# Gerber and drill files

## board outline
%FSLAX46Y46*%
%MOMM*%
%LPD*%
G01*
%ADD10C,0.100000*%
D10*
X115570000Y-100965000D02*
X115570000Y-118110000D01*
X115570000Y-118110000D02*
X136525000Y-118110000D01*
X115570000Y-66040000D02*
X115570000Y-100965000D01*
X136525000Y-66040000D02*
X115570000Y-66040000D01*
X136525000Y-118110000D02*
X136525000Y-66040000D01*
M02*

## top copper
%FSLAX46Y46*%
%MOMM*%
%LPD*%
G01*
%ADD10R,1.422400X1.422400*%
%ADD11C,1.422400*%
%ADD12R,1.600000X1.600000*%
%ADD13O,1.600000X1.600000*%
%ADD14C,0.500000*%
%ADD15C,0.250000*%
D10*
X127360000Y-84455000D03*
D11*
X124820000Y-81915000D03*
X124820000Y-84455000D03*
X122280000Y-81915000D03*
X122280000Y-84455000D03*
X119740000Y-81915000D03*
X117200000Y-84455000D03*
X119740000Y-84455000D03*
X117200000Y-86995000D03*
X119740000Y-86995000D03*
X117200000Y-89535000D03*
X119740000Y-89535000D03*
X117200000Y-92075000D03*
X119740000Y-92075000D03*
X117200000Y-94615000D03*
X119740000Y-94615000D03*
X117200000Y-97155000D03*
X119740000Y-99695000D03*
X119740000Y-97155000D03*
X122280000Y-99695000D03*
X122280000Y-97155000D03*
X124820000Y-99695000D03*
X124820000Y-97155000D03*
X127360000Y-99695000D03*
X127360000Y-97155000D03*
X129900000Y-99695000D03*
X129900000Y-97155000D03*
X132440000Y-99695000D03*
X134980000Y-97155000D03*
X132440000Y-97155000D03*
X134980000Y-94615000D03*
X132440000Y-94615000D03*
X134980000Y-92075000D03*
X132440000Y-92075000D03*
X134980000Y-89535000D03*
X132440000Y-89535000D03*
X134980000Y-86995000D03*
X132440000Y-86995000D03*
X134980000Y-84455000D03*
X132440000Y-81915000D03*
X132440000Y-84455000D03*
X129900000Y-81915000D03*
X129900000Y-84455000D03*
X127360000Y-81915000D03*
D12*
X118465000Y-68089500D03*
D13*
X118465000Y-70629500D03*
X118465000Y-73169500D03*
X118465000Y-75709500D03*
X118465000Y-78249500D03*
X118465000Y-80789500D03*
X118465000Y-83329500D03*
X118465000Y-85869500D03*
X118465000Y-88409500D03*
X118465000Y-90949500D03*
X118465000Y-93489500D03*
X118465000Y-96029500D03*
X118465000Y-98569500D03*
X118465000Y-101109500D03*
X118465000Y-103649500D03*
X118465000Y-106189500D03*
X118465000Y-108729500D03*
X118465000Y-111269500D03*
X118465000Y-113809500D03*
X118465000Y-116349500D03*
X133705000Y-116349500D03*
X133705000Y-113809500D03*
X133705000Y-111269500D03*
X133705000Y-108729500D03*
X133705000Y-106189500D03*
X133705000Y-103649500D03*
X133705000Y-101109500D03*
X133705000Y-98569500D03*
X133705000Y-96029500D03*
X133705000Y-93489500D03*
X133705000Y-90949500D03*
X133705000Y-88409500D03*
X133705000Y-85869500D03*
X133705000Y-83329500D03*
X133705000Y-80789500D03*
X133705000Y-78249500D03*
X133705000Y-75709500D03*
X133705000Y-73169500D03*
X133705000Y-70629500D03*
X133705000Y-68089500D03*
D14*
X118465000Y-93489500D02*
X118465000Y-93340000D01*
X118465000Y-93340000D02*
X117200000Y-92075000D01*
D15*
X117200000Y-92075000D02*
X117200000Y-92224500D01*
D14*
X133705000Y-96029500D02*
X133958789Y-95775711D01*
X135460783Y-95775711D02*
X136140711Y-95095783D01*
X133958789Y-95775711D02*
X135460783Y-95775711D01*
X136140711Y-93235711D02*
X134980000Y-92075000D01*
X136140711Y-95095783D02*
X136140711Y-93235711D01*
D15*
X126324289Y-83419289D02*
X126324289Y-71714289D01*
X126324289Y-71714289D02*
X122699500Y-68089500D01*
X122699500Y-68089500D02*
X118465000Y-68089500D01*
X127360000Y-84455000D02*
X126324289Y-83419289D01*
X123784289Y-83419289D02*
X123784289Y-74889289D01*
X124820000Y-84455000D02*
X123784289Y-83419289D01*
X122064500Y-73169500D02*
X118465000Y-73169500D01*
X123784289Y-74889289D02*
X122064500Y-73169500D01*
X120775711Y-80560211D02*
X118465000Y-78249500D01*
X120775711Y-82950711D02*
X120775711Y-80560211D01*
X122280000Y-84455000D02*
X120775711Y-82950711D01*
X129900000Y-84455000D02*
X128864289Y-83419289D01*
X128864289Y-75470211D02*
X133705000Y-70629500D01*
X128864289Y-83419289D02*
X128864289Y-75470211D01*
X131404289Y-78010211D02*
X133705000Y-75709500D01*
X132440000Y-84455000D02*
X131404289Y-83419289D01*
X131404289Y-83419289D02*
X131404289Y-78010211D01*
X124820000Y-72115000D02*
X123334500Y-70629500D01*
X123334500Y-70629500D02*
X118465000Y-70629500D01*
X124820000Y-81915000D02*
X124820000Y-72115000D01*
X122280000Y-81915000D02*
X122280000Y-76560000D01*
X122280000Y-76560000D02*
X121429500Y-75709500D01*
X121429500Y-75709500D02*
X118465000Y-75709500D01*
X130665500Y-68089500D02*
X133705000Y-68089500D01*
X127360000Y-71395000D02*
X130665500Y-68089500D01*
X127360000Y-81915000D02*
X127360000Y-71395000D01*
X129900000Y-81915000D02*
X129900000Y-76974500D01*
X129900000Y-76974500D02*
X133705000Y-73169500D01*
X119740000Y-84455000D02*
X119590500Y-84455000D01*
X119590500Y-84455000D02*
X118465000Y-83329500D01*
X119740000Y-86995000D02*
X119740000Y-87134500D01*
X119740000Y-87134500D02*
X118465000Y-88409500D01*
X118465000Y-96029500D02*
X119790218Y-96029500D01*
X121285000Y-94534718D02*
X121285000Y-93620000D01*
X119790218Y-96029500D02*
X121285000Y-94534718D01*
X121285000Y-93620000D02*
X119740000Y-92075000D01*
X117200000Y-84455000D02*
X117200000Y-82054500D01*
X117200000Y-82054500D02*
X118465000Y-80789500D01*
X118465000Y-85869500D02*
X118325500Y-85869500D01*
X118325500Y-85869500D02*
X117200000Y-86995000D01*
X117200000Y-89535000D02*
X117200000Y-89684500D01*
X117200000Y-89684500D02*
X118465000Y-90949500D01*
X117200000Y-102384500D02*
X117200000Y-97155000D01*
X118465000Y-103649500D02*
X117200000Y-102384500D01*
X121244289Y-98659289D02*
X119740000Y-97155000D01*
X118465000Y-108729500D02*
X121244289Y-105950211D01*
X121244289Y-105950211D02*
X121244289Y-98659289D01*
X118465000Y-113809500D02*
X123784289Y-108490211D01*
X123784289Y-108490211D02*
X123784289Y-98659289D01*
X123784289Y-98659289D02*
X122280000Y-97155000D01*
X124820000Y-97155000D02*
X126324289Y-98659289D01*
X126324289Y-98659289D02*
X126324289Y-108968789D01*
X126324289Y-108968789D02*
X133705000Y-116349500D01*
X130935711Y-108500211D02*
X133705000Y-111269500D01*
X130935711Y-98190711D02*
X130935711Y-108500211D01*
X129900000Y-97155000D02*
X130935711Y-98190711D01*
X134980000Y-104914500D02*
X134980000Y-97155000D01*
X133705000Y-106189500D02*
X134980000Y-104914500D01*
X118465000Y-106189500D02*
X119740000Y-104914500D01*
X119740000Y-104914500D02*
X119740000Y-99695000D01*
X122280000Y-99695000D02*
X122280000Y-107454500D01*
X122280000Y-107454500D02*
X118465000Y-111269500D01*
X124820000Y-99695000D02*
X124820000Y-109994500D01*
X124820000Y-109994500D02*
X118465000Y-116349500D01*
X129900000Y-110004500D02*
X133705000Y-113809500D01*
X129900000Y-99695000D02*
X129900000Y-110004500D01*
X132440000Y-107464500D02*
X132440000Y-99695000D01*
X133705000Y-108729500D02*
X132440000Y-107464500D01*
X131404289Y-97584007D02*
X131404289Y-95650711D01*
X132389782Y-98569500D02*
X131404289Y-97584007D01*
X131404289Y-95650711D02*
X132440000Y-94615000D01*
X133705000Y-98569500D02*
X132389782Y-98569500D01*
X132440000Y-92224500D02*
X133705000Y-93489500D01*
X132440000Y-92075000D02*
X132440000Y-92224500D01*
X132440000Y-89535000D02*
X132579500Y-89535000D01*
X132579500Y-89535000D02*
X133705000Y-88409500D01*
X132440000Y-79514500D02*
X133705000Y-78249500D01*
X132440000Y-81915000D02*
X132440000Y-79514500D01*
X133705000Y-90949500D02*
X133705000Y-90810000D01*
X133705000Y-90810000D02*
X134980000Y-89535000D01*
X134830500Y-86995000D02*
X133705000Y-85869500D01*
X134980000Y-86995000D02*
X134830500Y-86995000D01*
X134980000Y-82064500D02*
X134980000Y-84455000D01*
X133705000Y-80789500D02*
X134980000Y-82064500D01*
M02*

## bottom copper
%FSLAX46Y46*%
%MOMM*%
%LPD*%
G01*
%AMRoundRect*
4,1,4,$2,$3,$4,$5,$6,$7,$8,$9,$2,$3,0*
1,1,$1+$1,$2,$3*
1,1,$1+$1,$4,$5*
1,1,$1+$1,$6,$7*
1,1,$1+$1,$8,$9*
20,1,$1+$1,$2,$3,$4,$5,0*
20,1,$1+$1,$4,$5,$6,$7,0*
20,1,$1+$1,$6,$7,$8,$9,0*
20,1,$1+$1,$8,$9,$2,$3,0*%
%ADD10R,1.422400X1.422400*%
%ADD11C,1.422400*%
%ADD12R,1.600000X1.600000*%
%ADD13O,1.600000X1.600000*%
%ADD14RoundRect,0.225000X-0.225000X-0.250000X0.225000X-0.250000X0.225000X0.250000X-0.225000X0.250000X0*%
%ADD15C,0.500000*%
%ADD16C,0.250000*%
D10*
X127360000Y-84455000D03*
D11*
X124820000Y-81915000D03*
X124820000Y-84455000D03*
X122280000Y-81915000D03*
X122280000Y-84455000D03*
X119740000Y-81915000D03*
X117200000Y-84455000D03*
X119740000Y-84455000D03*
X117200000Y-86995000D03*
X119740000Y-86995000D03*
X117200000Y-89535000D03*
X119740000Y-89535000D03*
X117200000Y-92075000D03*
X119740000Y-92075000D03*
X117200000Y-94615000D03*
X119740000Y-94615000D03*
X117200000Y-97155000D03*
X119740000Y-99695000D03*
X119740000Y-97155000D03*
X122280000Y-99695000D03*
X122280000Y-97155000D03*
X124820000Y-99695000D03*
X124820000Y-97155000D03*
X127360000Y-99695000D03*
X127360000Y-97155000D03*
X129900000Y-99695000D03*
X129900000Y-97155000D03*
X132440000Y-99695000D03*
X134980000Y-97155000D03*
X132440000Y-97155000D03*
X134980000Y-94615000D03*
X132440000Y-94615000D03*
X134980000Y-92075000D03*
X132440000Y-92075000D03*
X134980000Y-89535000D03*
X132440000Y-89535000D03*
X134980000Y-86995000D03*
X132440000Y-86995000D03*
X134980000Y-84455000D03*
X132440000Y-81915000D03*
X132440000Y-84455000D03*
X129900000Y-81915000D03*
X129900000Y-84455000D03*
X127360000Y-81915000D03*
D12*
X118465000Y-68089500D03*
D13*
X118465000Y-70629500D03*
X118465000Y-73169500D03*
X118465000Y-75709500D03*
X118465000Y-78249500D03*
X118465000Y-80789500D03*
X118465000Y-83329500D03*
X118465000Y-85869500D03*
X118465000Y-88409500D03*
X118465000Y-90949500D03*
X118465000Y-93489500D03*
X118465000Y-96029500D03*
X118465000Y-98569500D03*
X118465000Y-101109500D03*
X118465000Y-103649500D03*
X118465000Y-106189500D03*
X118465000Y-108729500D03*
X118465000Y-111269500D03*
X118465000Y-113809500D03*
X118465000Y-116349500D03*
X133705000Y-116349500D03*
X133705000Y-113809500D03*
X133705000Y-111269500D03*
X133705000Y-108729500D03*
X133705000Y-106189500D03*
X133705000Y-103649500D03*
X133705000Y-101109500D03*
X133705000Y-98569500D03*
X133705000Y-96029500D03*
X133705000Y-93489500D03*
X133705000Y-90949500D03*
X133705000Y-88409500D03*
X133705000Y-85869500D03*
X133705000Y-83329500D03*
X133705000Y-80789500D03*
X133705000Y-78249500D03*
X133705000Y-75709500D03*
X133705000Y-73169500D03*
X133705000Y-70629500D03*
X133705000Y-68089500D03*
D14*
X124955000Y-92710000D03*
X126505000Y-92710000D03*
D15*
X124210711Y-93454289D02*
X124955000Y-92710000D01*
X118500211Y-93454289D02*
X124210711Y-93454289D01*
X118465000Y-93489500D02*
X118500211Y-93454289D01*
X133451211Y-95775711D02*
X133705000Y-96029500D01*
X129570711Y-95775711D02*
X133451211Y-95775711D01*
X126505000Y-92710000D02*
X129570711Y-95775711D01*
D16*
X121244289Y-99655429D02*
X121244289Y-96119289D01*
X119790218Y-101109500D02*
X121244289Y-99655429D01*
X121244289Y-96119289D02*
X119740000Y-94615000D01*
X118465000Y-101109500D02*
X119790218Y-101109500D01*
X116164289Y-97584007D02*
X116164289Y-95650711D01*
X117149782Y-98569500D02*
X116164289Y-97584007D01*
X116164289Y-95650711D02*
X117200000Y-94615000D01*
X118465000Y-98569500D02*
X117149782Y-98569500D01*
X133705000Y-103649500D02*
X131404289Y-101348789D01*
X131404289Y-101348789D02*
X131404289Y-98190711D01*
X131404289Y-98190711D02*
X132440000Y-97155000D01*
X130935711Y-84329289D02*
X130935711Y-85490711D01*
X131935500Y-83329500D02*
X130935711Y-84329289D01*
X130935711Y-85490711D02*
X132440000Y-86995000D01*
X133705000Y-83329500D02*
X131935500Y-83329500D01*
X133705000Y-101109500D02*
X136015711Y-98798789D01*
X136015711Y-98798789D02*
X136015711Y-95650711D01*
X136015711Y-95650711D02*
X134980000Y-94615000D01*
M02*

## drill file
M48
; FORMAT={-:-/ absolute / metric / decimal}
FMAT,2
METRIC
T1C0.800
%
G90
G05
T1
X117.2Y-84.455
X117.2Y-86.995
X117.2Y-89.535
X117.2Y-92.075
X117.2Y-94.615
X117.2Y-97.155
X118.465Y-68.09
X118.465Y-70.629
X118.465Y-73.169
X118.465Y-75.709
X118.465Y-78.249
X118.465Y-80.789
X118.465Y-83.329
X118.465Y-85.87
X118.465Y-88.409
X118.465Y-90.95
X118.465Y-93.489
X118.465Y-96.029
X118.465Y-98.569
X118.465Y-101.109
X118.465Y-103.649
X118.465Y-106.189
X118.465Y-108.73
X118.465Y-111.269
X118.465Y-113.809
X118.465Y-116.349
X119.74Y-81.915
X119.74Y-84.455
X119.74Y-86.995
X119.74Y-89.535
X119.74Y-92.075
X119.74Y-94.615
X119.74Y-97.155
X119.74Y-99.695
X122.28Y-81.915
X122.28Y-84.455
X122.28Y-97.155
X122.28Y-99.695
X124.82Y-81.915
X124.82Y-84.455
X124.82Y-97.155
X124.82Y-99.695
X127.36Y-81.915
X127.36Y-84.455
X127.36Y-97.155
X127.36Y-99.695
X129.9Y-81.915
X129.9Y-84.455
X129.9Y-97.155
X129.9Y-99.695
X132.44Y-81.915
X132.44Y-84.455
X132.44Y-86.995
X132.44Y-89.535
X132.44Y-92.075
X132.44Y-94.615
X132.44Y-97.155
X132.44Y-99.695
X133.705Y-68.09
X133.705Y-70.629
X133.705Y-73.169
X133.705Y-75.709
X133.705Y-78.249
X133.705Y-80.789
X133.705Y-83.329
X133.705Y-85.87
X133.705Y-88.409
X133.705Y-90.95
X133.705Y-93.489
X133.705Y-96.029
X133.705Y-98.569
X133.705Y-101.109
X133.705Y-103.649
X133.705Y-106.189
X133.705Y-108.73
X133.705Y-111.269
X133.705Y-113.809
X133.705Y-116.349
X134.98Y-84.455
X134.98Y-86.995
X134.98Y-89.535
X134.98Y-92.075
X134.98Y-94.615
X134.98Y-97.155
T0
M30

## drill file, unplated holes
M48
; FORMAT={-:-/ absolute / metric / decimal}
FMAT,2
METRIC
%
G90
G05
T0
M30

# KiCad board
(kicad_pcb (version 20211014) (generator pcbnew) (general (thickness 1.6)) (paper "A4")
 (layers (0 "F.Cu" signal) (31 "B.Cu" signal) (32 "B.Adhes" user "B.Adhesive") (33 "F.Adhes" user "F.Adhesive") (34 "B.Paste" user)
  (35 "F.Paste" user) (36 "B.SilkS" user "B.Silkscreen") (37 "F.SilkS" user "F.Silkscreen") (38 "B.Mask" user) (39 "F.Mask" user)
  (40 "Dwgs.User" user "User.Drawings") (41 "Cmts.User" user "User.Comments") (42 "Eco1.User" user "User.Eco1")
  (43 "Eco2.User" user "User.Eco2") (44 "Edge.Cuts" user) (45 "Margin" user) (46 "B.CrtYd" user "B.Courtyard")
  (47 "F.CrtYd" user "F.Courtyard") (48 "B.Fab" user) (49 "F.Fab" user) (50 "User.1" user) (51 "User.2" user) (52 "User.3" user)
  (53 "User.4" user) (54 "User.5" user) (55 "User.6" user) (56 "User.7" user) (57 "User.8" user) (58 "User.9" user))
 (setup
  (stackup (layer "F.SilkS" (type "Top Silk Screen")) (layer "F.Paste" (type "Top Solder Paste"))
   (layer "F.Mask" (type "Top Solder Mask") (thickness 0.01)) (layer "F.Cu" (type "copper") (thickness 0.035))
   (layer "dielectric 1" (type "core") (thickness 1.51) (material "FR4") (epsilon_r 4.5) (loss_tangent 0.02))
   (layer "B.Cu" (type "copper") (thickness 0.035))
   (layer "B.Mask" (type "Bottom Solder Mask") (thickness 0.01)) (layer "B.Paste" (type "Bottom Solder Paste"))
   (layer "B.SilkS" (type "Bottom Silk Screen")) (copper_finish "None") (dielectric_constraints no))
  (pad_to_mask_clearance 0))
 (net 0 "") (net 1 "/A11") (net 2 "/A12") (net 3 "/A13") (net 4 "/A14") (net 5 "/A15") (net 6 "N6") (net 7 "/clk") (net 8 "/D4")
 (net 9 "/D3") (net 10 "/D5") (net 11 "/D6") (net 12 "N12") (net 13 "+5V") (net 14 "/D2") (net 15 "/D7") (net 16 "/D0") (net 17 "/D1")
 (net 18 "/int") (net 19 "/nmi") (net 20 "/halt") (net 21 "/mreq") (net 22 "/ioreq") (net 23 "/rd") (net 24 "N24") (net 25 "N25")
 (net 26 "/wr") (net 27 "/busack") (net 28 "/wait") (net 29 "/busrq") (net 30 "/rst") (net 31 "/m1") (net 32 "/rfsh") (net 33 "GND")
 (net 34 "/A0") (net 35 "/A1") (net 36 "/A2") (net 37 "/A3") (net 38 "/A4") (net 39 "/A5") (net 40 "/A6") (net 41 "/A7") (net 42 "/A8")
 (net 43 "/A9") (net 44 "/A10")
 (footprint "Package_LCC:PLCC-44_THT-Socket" (layer "F.Cu") (at 127.36 84.455)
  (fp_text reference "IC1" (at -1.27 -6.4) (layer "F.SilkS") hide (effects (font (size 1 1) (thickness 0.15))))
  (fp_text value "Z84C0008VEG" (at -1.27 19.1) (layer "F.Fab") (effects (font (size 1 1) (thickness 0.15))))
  (pad "1" thru_hole rect locked (at 0 0) (size 1.4224 1.4224) (drill 0.8) (layers *.Cu *.Mask) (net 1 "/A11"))
  (pad "2" thru_hole circle locked (at -2.54 -2.54) (size 1.4224 1.4224) (drill 0.8) (layers *.Cu *.Mask) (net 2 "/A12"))
  (pad "3" thru_hole circle locked (at -2.54 0) (size 1.4224 1.4224) (drill 0.8) (layers *.Cu *.Mask) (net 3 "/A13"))
  (pad "4" thru_hole circle locked (at -5.08 -2.54) (size 1.4224 1.4224) (drill 0.8) (layers *.Cu *.Mask) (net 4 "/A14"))
  (pad "5" thru_hole circle locked (at -5.08 0) (size 1.4224 1.4224) (drill 0.8) (layers *.Cu *.Mask) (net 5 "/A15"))
  (pad "6" thru_hole circle locked (at -7.62 -2.54) (size 1.4224 1.4224) (drill 0.8) (layers *.Cu *.Mask) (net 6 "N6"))
  (pad "7" thru_hole circle locked (at -10.16 0) (size 1.4224 1.4224) (drill 0.8) (layers *.Cu *.Mask) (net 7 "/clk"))
  (pad "8" thru_hole circle locked (at -7.62 0) (size 1.4224 1.4224) (drill 0.8) (layers *.Cu *.Mask) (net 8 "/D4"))
  (pad "9" thru_hole circle locked (at -10.16 2.54) (size 1.4224 1.4224) (drill 0.8) (layers *.Cu *.Mask) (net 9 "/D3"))
  (pad "10" thru_hole circle locked (at -7.62 2.54) (size 1.4224 1.4224) (drill 0.8) (layers *.Cu *.Mask) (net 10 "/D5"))
  (pad "11" thru_hole circle locked (at -10.16 5.08) (size 1.4224 1.4224) (drill 0.8) (layers *.Cu *.Mask) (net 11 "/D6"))
  (pad "12" thru_hole circle locked (at -7.62 5.08) (size 1.4224 1.4224) (drill 0.8) (layers *.Cu *.Mask) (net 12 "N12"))
  (pad "13" thru_hole circle locked (at -10.16 7.62) (size 1.4224 1.4224) (drill 0.8) (layers *.Cu *.Mask) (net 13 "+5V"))
  (pad "14" thru_hole circle locked (at -7.62 7.62) (size 1.4224 1.4224) (drill 0.8) (layers *.Cu *.Mask) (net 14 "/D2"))
  (pad "15" thru_hole circle locked (at -10.16 10.16) (size 1.4224 1.4224) (drill 0.8) (layers *.Cu *.Mask) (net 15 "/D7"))
  (pad "16" thru_hole circle locked (at -7.62 10.16) (size 1.4224 1.4224) (drill 0.8) (layers *.Cu *.Mask) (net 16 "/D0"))
  (pad "17" thru_hole circle locked (at -10.16 12.7) (size 1.4224 1.4224) (drill 0.8) (layers *.Cu *.Mask) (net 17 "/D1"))
  (pad "18" thru_hole circle locked (at -7.62 15.24) (size 1.4224 1.4224) (drill 0.8) (layers *.Cu *.Mask) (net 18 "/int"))
  (pad "19" thru_hole circle locked (at -7.62 12.7) (size 1.4224 1.4224) (drill 0.8) (layers *.Cu *.Mask) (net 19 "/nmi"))
  (pad "20" thru_hole circle locked (at -5.08 15.24) (size 1.4224 1.4224) (drill 0.8) (layers *.Cu *.Mask) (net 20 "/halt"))
  (pad "21" thru_hole circle locked (at -5.08 12.7) (size 1.4224 1.4224) (drill 0.8) (layers *.Cu *.Mask) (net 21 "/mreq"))
  (pad "22" thru_hole circle locked (at -2.54 15.24) (size 1.4224 1.4224) (drill 0.8) (layers *.Cu *.Mask) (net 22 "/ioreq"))
  (pad "23" thru_hole circle locked (at -2.54 12.7) (size 1.4224 1.4224) (drill 0.8) (layers *.Cu *.Mask) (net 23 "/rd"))
  (pad "24" thru_hole circle locked (at 0 15.24) (size 1.4224 1.4224) (drill 0.8) (layers *.Cu *.Mask) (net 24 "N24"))
  (pad "25" thru_hole circle locked (at 0 12.7) (size 1.4224 1.4224) (drill 0.8) (layers *.Cu *.Mask) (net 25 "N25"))
  (pad "26" thru_hole circle locked (at 2.54 15.24) (size 1.4224 1.4224) (drill 0.8) (layers *.Cu *.Mask) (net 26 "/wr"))
  (pad "27" thru_hole circle locked (at 2.54 12.7) (size 1.4224 1.4224) (drill 0.8) (layers *.Cu *.Mask) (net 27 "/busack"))
  (pad "28" thru_hole circle locked (at 5.08 15.24) (size 1.4224 1.4224) (drill 0.8) (layers *.Cu *.Mask) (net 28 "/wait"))
  (pad "29" thru_hole circle locked (at 7.62 12.7) (size 1.4224 1.4224) (drill 0.8) (layers *.Cu *.Mask) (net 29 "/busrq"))
  (pad "30" thru_hole circle locked (at 5.08 12.7) (size 1.4224 1.4224) (drill 0.8) (layers *.Cu *.Mask) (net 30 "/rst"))
  (pad "31" thru_hole circle locked (at 7.62 10.16) (size 1.4224 1.4224) (drill 0.8) (layers *.Cu *.Mask) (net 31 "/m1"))
  (pad "32" thru_hole circle locked (at 5.08 10.16) (size 1.4224 1.4224) (drill 0.8) (layers *.Cu *.Mask) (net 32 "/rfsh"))
  (pad "33" thru_hole circle locked (at 7.62 7.62) (size 1.4224 1.4224) (drill 0.8) (layers *.Cu *.Mask) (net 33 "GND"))
  (pad "34" thru_hole circle locked (at 5.08 7.62) (size 1.4224 1.4224) (drill 0.8) (layers *.Cu *.Mask) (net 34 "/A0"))
  (pad "35" thru_hole circle locked (at 7.62 5.08) (size 1.4224 1.4224) (drill 0.8) (layers *.Cu *.Mask) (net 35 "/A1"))
  (pad "36" thru_hole circle locked (at 5.08 5.08) (size 1.4224 1.4224) (drill 0.8) (layers *.Cu *.Mask) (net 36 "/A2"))
  (pad "37" thru_hole circle locked (at 7.62 2.54) (size 1.4224 1.4224) (drill 0.8) (layers *.Cu *.Mask) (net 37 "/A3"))
  (pad "38" thru_hole circle locked (at 5.08 2.54) (size 1.4224 1.4224) (drill 0.8) (layers *.Cu *.Mask) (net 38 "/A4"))
  (pad "39" thru_hole circle locked (at 7.62 0) (size 1.4224 1.4224) (drill 0.8) (layers *.Cu *.Mask) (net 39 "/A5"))
  (pad "40" thru_hole circle locked (at 5.08 -2.54) (size 1.4224 1.4224) (drill 0.8) (layers *.Cu *.Mask) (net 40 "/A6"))
  (pad "41" thru_hole circle locked (at 5.08 0) (size 1.4224 1.4224) (drill 0.8) (layers *.Cu *.Mask) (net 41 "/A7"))
  (pad "42" thru_hole circle locked (at 2.54 -2.54) (size 1.4224 1.4224) (drill 0.8) (layers *.Cu *.Mask) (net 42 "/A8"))
  (pad "43" thru_hole circle locked (at 2.54 0) (size 1.4224 1.4224) (drill 0.8) (layers *.Cu *.Mask) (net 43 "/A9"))
  (pad "44" thru_hole circle locked (at 0 -2.54) (size 1.4224 1.4224) (drill 0.8) (layers *.Cu *.Mask) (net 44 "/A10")))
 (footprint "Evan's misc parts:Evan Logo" (layer "F.Cu") (at 125.73 111.125)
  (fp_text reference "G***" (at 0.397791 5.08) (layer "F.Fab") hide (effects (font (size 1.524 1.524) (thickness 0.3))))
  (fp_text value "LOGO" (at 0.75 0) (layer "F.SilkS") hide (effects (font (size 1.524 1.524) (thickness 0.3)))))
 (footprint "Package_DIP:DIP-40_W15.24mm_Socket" (layer "F.Cu") (at 118.465 68.0895)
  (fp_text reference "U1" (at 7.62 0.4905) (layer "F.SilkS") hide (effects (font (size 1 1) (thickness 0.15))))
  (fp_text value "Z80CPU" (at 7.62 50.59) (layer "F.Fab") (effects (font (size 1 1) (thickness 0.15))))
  (pad "1" thru_hole rect locked (at 0 0) (size 1.6 1.6) (drill 0.8) (layers *.Cu *.Mask) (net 1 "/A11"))
  (pad "2" thru_hole oval locked (at 0 2.54) (size 1.6 1.6) (drill 0.8) (layers *.Cu *.Mask) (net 2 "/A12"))
  (pad "3" thru_hole oval locked (at 0 5.08) (size 1.6 1.6) (drill 0.8) (layers *.Cu *.Mask) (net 3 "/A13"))
  (pad "4" thru_hole oval locked (at 0 7.62) (size 1.6 1.6) (drill 0.8) (layers *.Cu *.Mask) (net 4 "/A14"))
  (pad "5" thru_hole oval locked (at 0 10.16) (size 1.6 1.6) (drill 0.8) (layers *.Cu *.Mask) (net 5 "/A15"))
  (pad "6" thru_hole oval locked (at 0 12.7) (size 1.6 1.6) (drill 0.8) (layers *.Cu *.Mask) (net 7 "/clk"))
  (pad "7" thru_hole oval locked (at 0 15.24) (size 1.6 1.6) (drill 0.8) (layers *.Cu *.Mask) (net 8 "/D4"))
  (pad "8" thru_hole oval locked (at 0 17.78) (size 1.6 1.6) (drill 0.8) (layers *.Cu *.Mask) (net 9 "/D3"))
  (pad "9" thru_hole oval locked (at 0 20.32) (size 1.6 1.6) (drill 0.8) (layers *.Cu *.Mask) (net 10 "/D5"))
  (pad "10" thru_hole oval locked (at 0 22.86) (size 1.6 1.6) (drill 0.8) (layers *.Cu *.Mask) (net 11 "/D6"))
  (pad "11" thru_hole oval locked (at 0 25.4) (size 1.6 1.6) (drill 0.8) (layers *.Cu *.Mask) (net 13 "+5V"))
  (pad "12" thru_hole oval locked (at 0 27.94) (size 1.6 1.6) (drill 0.8) (layers *.Cu *.Mask) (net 14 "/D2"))
  (pad "13" thru_hole oval locked (at 0 30.48) (size 1.6 1.6) (drill 0.8) (layers *.Cu *.Mask) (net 15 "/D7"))
  (pad "14" thru_hole oval locked (at 0 33.02) (size 1.6 1.6) (drill 0.8) (layers *.Cu *.Mask) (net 16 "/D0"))
  (pad "15" thru_hole oval locked (at 0 35.56) (size 1.6 1.6) (drill 0.8) (layers *.Cu *.Mask) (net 17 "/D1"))
  (pad "16" thru_hole oval locked (at 0 38.1) (size 1.6 1.6) (drill 0.8) (layers *.Cu *.Mask) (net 18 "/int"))
  (pad "17" thru_hole oval locked (at 0 40.64) (size 1.6 1.6) (drill 0.8) (layers *.Cu *.Mask) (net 19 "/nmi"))
  (pad "18" thru_hole oval locked (at 0 43.18) (size 1.6 1.6) (drill 0.8) (layers *.Cu *.Mask) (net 20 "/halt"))
  (pad "19" thru_hole oval locked (at 0 45.72) (size 1.6 1.6) (drill 0.8) (layers *.Cu *.Mask) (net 21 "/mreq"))
  (pad "20" thru_hole oval locked (at 0 48.26) (size 1.6 1.6) (drill 0.8) (layers *.Cu *.Mask) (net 22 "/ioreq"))
  (pad "21" thru_hole oval locked (at 15.24 48.26) (size 1.6 1.6) (drill 0.8) (layers *.Cu *.Mask) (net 23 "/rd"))
  (pad "22" thru_hole oval locked (at 15.24 45.72) (size 1.6 1.6) (drill 0.8) (layers *.Cu *.Mask) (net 26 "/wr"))
  (pad "23" thru_hole oval locked (at 15.24 43.18) (size 1.6 1.6) (drill 0.8) (layers *.Cu *.Mask) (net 27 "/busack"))
  (pad "24" thru_hole oval locked (at 15.24 40.64) (size 1.6 1.6) (drill 0.8) (layers *.Cu *.Mask) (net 28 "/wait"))
  (pad "25" thru_hole oval locked (at 15.24 38.1) (size 1.6 1.6) (drill 0.8) (layers *.Cu *.Mask) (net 29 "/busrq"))
  (pad "26" thru_hole oval locked (at 15.24 35.56) (size 1.6 1.6) (drill 0.8) (layers *.Cu *.Mask) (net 30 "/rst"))
  (pad "27" thru_hole oval locked (at 15.24 33.02) (size 1.6 1.6) (drill 0.8) (layers *.Cu *.Mask) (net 31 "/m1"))
  (pad "28" thru_hole oval locked (at 15.24 30.48) (size 1.6 1.6) (drill 0.8) (layers *.Cu *.Mask) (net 32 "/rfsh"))
  (pad "29" thru_hole oval locked (at 15.24 27.94) (size 1.6 1.6) (drill 0.8) (layers *.Cu *.Mask) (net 33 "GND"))
  (pad "30" thru_hole oval locked (at 15.24 25.4) (size 1.6 1.6) (drill 0.8) (layers *.Cu *.Mask) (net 34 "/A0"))
  (pad "31" thru_hole oval locked (at 15.24 22.86) (size 1.6 1.6) (drill 0.8) (layers *.Cu *.Mask) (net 35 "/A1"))
  (pad "32" thru_hole oval locked (at 15.24 20.32) (size 1.6 1.6) (drill 0.8) (layers *.Cu *.Mask) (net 36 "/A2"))
  (pad "33" thru_hole oval locked (at 15.24 17.78) (size 1.6 1.6) (drill 0.8) (layers *.Cu *.Mask) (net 37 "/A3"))
  (pad "34" thru_hole oval locked (at 15.24 15.24) (size 1.6 1.6) (drill 0.8) (layers *.Cu *.Mask) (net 38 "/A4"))
  (pad "35" thru_hole oval locked (at 15.24 12.7) (size 1.6 1.6) (drill 0.8) (layers *.Cu *.Mask) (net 39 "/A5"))
  (pad "36" thru_hole oval locked (at 15.24 10.16) (size 1.6 1.6) (drill 0.8) (layers *.Cu *.Mask) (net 40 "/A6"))
  (pad "37" thru_hole oval locked (at 15.24 7.62) (size 1.6 1.6) (drill 0.8) (layers *.Cu *.Mask) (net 41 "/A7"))
  (pad "38" thru_hole oval locked (at 15.24 5.08) (size 1.6 1.6) (drill 0.8) (layers *.Cu *.Mask) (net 42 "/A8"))
  (pad "39" thru_hole oval locked (at 15.24 2.54) (size 1.6 1.6) (drill 0.8) (layers *.Cu *.Mask) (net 43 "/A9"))
  (pad "40" thru_hole oval locked (at 15.24 0) (size 1.6 1.6) (drill 0.8) (layers *.Cu *.Mask) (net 44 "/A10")))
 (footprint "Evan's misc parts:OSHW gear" (layer "B.Cu") (at 125.73 110.49 180)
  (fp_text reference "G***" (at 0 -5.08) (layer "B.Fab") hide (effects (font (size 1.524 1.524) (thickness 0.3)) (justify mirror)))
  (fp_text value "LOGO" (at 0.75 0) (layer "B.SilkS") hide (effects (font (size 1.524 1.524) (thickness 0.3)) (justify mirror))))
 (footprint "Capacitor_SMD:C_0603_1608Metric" (layer "B.Cu") (at 125.73 92.71)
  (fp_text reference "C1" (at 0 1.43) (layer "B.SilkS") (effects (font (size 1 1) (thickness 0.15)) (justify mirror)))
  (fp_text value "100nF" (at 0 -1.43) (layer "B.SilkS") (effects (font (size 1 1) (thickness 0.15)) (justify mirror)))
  (pad "1" smd roundrect locked (at -0.775 0) (size 0.9 0.95) (layers "B.Cu" "B.Paste" "B.Mask") (roundrect_rratio 0.25) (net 13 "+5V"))
  (pad "2" smd roundrect locked (at 0.775 0) (size 0.9 0.95) (layers "B.Cu" "B.Paste" "B.Mask") (roundrect_rratio 0.25) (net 33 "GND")))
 (gr_line (start 115.57 100.965) (end 115.57 118.11) (layer "Edge.Cuts") (width 0.1))
 (gr_line (start 115.57 118.11) (end 136.525 118.11) (layer "Edge.Cuts") (width 0.1))
 (gr_line (start 115.57 66.04) (end 115.57 100.965) (layer "Edge.Cuts") (width 0.1))
 (gr_line (start 136.525 66.04) (end 115.57 66.04) (layer "Edge.Cuts") (width 0.1))
 (gr_line (start 136.525 118.11) (end 136.525 66.04) (layer "Edge.Cuts") (width 0.1))
 (segment (start 118.465 93.4895) (end 118.465 93.34) (width 0.5) (layer "F.Cu") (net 13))
 (segment (start 118.465 93.34) (end 117.2 92.075) (width 0.5) (layer "F.Cu") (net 13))
 (segment (start 117.2 92.075) (end 117.2 92.2245) (width 0.25) (layer "F.Cu") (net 13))
 (segment (start 124.210711 93.454289) (end 124.955 92.71) (width 0.5) (layer "B.Cu") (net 13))
 (segment (start 118.500211 93.454289) (end 124.210711 93.454289) (width 0.5) (layer "B.Cu") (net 13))
 (segment (start 118.465 93.4895) (end 118.500211 93.454289) (width 0.5) (layer "B.Cu") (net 13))
 (segment (start 133.705 96.0295) (end 133.958789 95.775711) (width 0.5) (layer "F.Cu") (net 33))
 (segment (start 135.460783 95.775711) (end 136.140711 95.095783) (width 0.5) (layer "F.Cu") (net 33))
 (segment (start 133.958789 95.775711) (end 135.460783 95.775711) (width 0.5) (layer "F.Cu") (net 33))
 (segment (start 136.140711 93.235711) (end 134.98 92.075) (width 0.5) (layer "F.Cu") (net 33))
 (segment (start 136.140711 95.095783) (end 136.140711 93.235711) (width 0.5) (layer "F.Cu") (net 33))
 (segment (start 133.451211 95.775711) (end 133.705 96.0295) (width 0.5) (layer "B.Cu") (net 33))
 (segment (start 129.570711 95.775711) (end 133.451211 95.775711) (width 0.5) (layer "B.Cu") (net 33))
 (segment (start 126.505 92.71) (end 129.570711 95.775711) (width 0.5) (layer "B.Cu") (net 33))
 (segment (start 126.324289 83.419289) (end 126.324289 71.714289) (width 0.25) (layer "F.Cu") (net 1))
 (segment (start 126.324289 71.714289) (end 122.6995 68.0895) (width 0.25) (layer "F.Cu") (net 1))
 (segment (start 122.6995 68.0895) (end 118.465 68.0895) (width 0.25) (layer "F.Cu") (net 1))
 (segment (start 127.36 84.455) (end 126.324289 83.419289) (width 0.25) (layer "F.Cu") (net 1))
 (segment (start 123.784289 83.419289) (end 123.784289 74.889289) (width 0.25) (layer "F.Cu") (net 3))
 (segment (start 124.82 84.455) (end 123.784289 83.419289) (width 0.25) (layer "F.Cu") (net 3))
 (segment (start 122.0645 73.1695) (end 118.465 73.1695) (width 0.25) (layer "F.Cu") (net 3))
 (segment (start 123.784289 74.889289) (end 122.0645 73.1695) (width 0.25) (layer "F.Cu") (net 3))
 (segment (start 120.775711 80.560211) (end 118.465 78.2495) (width 0.25) (layer "F.Cu") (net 5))
 (segment (start 120.775711 82.950711) (end 120.775711 80.560211) (width 0.25) (layer "F.Cu") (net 5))
 (segment (start 122.28 84.455) (end 120.775711 82.950711) (width 0.25) (layer "F.Cu") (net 5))
 (segment (start 129.9 84.455) (end 128.864289 83.419289) (width 0.25) (layer "F.Cu") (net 43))
 (segment (start 128.864289 75.470211) (end 133.705 70.6295) (width 0.25) (layer "F.Cu") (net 43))
 (segment (start 128.864289 83.419289) (end 128.864289 75.470211) (width 0.25) (layer "F.Cu") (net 43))
 (segment (start 131.404289 78.010211) (end 133.705 75.7095) (width 0.25) (layer "F.Cu") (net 41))
 (segment (start 132.44 84.455) (end 131.404289 83.419289) (width 0.25) (layer "F.Cu") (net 41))
 (segment (start 131.404289 83.419289) (end 131.404289 78.010211) (width 0.25) (layer "F.Cu") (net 41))
 (segment (start 124.82 72.115) (end 123.3345 70.6295) (width 0.25) (layer "F.Cu") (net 2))
 (segment (start 123.3345 70.6295) (end 118.465 70.6295) (width 0.25) (layer "F.Cu") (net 2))
 (segment (start 124.82 81.915) (end 124.82 72.115) (width 0.25) (layer "F.Cu") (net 2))
 (segment (start 122.28 81.915) (end 122.28 76.56) (width 0.25) (layer "F.Cu") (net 4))
 (segment (start 122.28 76.56) (end 121.4295 75.7095) (width 0.25) (layer "F.Cu") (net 4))
 (segment (start 121.4295 75.7095) (end 118.465 75.7095) (width 0.25) (layer "F.Cu") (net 4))
 (segment (start 130.6655 68.0895) (end 133.705 68.0895) (width 0.25) (layer "F.Cu") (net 44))
 (segment (start 127.36 71.395) (end 130.6655 68.0895) (width 0.25) (layer "F.Cu") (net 44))
 (segment (start 127.36 81.915) (end 127.36 71.395) (width 0.25) (layer "F.Cu") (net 44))
 (segment (start 129.9 81.915) (end 129.9 76.9745) (width 0.25) (layer "F.Cu") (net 42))
 (segment (start 129.9 76.9745) (end 133.705 73.1695) (width 0.25) (layer "F.Cu") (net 42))
 (segment (start 119.74 84.455) (end 119.5905 84.455) (width 0.25) (layer "F.Cu") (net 8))
 (segment (start 119.5905 84.455) (end 118.465 83.3295) (width 0.25) (layer "F.Cu") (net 8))
 (segment (start 119.74 86.995) (end 119.74 87.1345) (width 0.25) (layer "F.Cu") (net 10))
 (segment (start 119.74 87.1345) (end 118.465 88.4095) (width 0.25) (layer "F.Cu") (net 10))
 (segment (start 118.465 96.0295) (end 119.790218 96.0295) (width 0.25) (layer "F.Cu") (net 14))
 (segment (start 121.285 94.534718) (end 121.285 93.62) (width 0.25) (layer "F.Cu") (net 14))
 (segment (start 119.790218 96.0295) (end 121.285 94.534718) (width 0.25) (layer "F.Cu") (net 14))
 (segment (start 121.285 93.62) (end 119.74 92.075) (width 0.25) (layer "F.Cu") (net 14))
 (segment (start 121.244289 99.655429) (end 121.244289 96.119289) (width 0.25) (layer "B.Cu") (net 16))
 (segment (start 119.790218 101.1095) (end 121.244289 99.655429) (width 0.25) (layer "B.Cu") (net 16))
 (segment (start 121.244289 96.119289) (end 119.74 94.615) (width 0.25) (layer "B.Cu") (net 16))
 (segment (start 118.465 101.1095) (end 119.790218 101.1095) (width 0.25) (layer "B.Cu") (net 16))
 (segment (start 117.2 84.455) (end 117.2 82.0545) (width 0.25) (layer "F.Cu") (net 7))
 (segment (start 117.2 82.0545) (end 118.465 80.7895) (width 0.25) (layer "F.Cu") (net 7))
 (segment (start 118.465 85.8695) (end 118.3255 85.8695) (width 0.25) (layer "F.Cu") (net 9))
 (segment (start 118.3255 85.8695) (end 117.2 86.995) (width 0.25) (layer "F.Cu") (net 9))
 (segment (start 117.2 89.535) (end 117.2 89.6845) (width 0.25) (layer "F.Cu") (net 11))
 (segment (start 117.2 89.6845) (end 118.465 90.9495) (width 0.25) (layer "F.Cu") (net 11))
 (segment (start 116.164289 97.584007) (end 116.164289 95.650711) (width 0.25) (layer "B.Cu") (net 15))
 (segment (start 117.149782 98.5695) (end 116.164289 97.584007) (width 0.25) (layer "B.Cu") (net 15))
 (segment (start 116.164289 95.650711) (end 117.2 94.615) (width 0.25) (layer "B.Cu") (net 15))
 (segment (start 118.465 98.5695) (end 117.149782 98.5695) (width 0.25) (layer "B.Cu") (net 15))
 (segment (start 117.2 102.3845) (end 117.2 97.155) (width 0.25) (layer "F.Cu") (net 17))
 (segment (start 118.465 103.6495) (end 117.2 102.3845) (width 0.25) (layer "F.Cu") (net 17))
 (segment (start 121.244289 98.659289) (end 119.74 97.155) (width 0.25) (layer "F.Cu") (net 19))
 (segment (start 118.465 108.7295) (end 121.244289 105.950211) (width 0.25) (layer "F.Cu") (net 19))
 (segment (start 121.244289 105.950211) (end 121.244289 98.659289) (width 0.25) (layer "F.Cu") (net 19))
 (segment (start 118.465 113.8095) (end 123.784289 108.490211) (width 0.25) (layer "F.Cu") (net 21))
 (segment (start 123.784289 108.490211) (end 123.784289 98.659289) (width 0.25) (layer "F.Cu") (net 21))
 (segment (start 123.784289 98.659289) (end 122.28 97.155) (width 0.25) (layer "F.Cu") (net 21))
 (segment (start 124.82 97.155) (end 126.324289 98.659289) (width 0.25) (layer "F.Cu") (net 23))
 (segment (start 126.324289 98.659289) (end 126.324289 108.968789) (width 0.25) (layer "F.Cu") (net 23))
 (segment (start 126.324289 108.968789) (end 133.705 116.3495) (width 0.25) (layer "F.Cu") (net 23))
 (segment (start 130.935711 108.500211) (end 133.705 111.2695) (width 0.25) (layer "F.Cu") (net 27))
 (segment (start 130.935711 98.190711) (end 130.935711 108.500211) (width 0.25) (layer "F.Cu") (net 27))
 (segment (start 129.9 97.155) (end 130.935711 98.190711) (width 0.25) (layer "F.Cu") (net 27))
 (segment (start 134.98 104.9145) (end 134.98 97.155) (width 0.25) (layer "F.Cu") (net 29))
 (segment (start 133.705 106.1895) (end 134.98 104.9145) (width 0.25) (layer "F.Cu") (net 29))
 (segment (start 118.465 106.1895) (end 119.74 104.9145) (width 0.25) (layer "F.Cu") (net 18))
 (segment (start 119.74 104.9145) (end 119.74 99.695) (width 0.25) (layer "F.Cu") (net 18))
 (segment (start 122.28 99.695) (end 122.28 107.4545) (width 0.25) (layer "F.Cu") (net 20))
 (segment (start 122.28 107.4545) (end 118.465 111.2695) (width 0.25) (layer "F.Cu") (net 20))
 (segment (start 124.82 99.695) (end 124.82 109.9945) (width 0.25) (layer "F.Cu") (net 22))
 (segment (start 124.82 109.9945) (end 118.465 116.3495) (width 0.25) (layer "F.Cu") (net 22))
 (segment (start 129.9 110.0045) (end 133.705 113.8095) (width 0.25) (layer "F.Cu") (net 26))
 (segment (start 129.9 99.695) (end 129.9 110.0045) (width 0.25) (layer "F.Cu") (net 26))
 (segment (start 132.44 107.4645) (end 132.44 99.695) (width 0.25) (layer "F.Cu") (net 28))
 (segment (start 133.705 108.7295) (end 132.44 107.4645) (width 0.25) (layer "F.Cu") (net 28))
 (segment (start 133.705 103.6495) (end 131.404289 101.348789) (width 0.25) (layer "B.Cu") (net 30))
 (segment (start 131.404289 101.348789) (end 131.404289 98.190711) (width 0.25) (layer "B.Cu") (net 30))
 (segment (start 131.404289 98.190711) (end 132.44 97.155) (width 0.25) (layer "B.Cu") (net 30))
 (segment (start 131.404289 97.584007) (end 131.404289 95.650711) (width 0.25) (layer "F.Cu") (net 32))
 (segment (start 132.389782 98.5695) (end 131.404289 97.584007) (width 0.25) (layer "F.Cu") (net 32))
 (segment (start 131.404289 95.650711) (end 132.44 94.615) (width 0.25) (layer "F.Cu") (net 32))
 (segment (start 133.705 98.5695) (end 132.389782 98.5695) (width 0.25) (layer "F.Cu") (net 32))
 (segment (start 132.44 92.2245) (end 133.705 93.4895) (width 0.25) (layer "F.Cu") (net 34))
 (segment (start 132.44 92.075) (end 132.44 92.2245) (width 0.25) (layer "F.Cu") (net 34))
 (segment (start 132.44 89.535) (end 132.5795 89.535) (width 0.25) (layer "F.Cu") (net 36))
 (segment (start 132.5795 89.535) (end 133.705 88.4095) (width 0.25) (layer "F.Cu") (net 36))
 (segment (start 130.935711 84.329289) (end 130.935711 85.490711) (width 0.25) (layer "B.Cu") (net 38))
 (segment (start 131.9355 83.3295) (end 130.935711 84.329289) (width 0.25) (layer "B.Cu") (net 38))
 (segment (start 130.935711 85.490711) (end 132.44 86.995) (width 0.25) (layer "B.Cu") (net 38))
 (segment (start 133.705 83.3295) (end 131.9355 83.3295) (width 0.25) (layer "B.Cu") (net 38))
 (segment (start 132.44 79.5145) (end 133.705 78.2495) (width 0.25) (layer "F.Cu") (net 40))
 (segment (start 132.44 81.915) (end 132.44 79.5145) (width 0.25) (layer "F.Cu") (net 40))
 (segment (start 133.705 101.1095) (end 136.015711 98.798789) (width 0.25) (layer "B.Cu") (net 31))
 (segment (start 136.015711 98.798789) (end 136.015711 95.650711) (width 0.25) (layer "B.Cu") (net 31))
 (segment (start 136.015711 95.650711) (end 134.98 94.615) (width 0.25) (layer "B.Cu") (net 31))
 (segment (start 133.705 90.9495) (end 133.705 90.81) (width 0.25) (layer "F.Cu") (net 35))
 (segment (start 133.705 90.81) (end 134.98 89.535) (width 0.25) (layer "F.Cu") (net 35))
 (segment (start 134.8305 86.995) (end 133.705 85.8695) (width 0.25) (layer "F.Cu") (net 37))
 (segment (start 134.98 86.995) (end 134.8305 86.995) (width 0.25) (layer "F.Cu") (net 37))
 (segment (start 134.98 82.0645) (end 134.98 84.455) (width 0.25) (layer "F.Cu") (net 39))
 (segment (start 133.705 80.7895) (end 134.98 82.0645) (width 0.25) (layer "F.Cu") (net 39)))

